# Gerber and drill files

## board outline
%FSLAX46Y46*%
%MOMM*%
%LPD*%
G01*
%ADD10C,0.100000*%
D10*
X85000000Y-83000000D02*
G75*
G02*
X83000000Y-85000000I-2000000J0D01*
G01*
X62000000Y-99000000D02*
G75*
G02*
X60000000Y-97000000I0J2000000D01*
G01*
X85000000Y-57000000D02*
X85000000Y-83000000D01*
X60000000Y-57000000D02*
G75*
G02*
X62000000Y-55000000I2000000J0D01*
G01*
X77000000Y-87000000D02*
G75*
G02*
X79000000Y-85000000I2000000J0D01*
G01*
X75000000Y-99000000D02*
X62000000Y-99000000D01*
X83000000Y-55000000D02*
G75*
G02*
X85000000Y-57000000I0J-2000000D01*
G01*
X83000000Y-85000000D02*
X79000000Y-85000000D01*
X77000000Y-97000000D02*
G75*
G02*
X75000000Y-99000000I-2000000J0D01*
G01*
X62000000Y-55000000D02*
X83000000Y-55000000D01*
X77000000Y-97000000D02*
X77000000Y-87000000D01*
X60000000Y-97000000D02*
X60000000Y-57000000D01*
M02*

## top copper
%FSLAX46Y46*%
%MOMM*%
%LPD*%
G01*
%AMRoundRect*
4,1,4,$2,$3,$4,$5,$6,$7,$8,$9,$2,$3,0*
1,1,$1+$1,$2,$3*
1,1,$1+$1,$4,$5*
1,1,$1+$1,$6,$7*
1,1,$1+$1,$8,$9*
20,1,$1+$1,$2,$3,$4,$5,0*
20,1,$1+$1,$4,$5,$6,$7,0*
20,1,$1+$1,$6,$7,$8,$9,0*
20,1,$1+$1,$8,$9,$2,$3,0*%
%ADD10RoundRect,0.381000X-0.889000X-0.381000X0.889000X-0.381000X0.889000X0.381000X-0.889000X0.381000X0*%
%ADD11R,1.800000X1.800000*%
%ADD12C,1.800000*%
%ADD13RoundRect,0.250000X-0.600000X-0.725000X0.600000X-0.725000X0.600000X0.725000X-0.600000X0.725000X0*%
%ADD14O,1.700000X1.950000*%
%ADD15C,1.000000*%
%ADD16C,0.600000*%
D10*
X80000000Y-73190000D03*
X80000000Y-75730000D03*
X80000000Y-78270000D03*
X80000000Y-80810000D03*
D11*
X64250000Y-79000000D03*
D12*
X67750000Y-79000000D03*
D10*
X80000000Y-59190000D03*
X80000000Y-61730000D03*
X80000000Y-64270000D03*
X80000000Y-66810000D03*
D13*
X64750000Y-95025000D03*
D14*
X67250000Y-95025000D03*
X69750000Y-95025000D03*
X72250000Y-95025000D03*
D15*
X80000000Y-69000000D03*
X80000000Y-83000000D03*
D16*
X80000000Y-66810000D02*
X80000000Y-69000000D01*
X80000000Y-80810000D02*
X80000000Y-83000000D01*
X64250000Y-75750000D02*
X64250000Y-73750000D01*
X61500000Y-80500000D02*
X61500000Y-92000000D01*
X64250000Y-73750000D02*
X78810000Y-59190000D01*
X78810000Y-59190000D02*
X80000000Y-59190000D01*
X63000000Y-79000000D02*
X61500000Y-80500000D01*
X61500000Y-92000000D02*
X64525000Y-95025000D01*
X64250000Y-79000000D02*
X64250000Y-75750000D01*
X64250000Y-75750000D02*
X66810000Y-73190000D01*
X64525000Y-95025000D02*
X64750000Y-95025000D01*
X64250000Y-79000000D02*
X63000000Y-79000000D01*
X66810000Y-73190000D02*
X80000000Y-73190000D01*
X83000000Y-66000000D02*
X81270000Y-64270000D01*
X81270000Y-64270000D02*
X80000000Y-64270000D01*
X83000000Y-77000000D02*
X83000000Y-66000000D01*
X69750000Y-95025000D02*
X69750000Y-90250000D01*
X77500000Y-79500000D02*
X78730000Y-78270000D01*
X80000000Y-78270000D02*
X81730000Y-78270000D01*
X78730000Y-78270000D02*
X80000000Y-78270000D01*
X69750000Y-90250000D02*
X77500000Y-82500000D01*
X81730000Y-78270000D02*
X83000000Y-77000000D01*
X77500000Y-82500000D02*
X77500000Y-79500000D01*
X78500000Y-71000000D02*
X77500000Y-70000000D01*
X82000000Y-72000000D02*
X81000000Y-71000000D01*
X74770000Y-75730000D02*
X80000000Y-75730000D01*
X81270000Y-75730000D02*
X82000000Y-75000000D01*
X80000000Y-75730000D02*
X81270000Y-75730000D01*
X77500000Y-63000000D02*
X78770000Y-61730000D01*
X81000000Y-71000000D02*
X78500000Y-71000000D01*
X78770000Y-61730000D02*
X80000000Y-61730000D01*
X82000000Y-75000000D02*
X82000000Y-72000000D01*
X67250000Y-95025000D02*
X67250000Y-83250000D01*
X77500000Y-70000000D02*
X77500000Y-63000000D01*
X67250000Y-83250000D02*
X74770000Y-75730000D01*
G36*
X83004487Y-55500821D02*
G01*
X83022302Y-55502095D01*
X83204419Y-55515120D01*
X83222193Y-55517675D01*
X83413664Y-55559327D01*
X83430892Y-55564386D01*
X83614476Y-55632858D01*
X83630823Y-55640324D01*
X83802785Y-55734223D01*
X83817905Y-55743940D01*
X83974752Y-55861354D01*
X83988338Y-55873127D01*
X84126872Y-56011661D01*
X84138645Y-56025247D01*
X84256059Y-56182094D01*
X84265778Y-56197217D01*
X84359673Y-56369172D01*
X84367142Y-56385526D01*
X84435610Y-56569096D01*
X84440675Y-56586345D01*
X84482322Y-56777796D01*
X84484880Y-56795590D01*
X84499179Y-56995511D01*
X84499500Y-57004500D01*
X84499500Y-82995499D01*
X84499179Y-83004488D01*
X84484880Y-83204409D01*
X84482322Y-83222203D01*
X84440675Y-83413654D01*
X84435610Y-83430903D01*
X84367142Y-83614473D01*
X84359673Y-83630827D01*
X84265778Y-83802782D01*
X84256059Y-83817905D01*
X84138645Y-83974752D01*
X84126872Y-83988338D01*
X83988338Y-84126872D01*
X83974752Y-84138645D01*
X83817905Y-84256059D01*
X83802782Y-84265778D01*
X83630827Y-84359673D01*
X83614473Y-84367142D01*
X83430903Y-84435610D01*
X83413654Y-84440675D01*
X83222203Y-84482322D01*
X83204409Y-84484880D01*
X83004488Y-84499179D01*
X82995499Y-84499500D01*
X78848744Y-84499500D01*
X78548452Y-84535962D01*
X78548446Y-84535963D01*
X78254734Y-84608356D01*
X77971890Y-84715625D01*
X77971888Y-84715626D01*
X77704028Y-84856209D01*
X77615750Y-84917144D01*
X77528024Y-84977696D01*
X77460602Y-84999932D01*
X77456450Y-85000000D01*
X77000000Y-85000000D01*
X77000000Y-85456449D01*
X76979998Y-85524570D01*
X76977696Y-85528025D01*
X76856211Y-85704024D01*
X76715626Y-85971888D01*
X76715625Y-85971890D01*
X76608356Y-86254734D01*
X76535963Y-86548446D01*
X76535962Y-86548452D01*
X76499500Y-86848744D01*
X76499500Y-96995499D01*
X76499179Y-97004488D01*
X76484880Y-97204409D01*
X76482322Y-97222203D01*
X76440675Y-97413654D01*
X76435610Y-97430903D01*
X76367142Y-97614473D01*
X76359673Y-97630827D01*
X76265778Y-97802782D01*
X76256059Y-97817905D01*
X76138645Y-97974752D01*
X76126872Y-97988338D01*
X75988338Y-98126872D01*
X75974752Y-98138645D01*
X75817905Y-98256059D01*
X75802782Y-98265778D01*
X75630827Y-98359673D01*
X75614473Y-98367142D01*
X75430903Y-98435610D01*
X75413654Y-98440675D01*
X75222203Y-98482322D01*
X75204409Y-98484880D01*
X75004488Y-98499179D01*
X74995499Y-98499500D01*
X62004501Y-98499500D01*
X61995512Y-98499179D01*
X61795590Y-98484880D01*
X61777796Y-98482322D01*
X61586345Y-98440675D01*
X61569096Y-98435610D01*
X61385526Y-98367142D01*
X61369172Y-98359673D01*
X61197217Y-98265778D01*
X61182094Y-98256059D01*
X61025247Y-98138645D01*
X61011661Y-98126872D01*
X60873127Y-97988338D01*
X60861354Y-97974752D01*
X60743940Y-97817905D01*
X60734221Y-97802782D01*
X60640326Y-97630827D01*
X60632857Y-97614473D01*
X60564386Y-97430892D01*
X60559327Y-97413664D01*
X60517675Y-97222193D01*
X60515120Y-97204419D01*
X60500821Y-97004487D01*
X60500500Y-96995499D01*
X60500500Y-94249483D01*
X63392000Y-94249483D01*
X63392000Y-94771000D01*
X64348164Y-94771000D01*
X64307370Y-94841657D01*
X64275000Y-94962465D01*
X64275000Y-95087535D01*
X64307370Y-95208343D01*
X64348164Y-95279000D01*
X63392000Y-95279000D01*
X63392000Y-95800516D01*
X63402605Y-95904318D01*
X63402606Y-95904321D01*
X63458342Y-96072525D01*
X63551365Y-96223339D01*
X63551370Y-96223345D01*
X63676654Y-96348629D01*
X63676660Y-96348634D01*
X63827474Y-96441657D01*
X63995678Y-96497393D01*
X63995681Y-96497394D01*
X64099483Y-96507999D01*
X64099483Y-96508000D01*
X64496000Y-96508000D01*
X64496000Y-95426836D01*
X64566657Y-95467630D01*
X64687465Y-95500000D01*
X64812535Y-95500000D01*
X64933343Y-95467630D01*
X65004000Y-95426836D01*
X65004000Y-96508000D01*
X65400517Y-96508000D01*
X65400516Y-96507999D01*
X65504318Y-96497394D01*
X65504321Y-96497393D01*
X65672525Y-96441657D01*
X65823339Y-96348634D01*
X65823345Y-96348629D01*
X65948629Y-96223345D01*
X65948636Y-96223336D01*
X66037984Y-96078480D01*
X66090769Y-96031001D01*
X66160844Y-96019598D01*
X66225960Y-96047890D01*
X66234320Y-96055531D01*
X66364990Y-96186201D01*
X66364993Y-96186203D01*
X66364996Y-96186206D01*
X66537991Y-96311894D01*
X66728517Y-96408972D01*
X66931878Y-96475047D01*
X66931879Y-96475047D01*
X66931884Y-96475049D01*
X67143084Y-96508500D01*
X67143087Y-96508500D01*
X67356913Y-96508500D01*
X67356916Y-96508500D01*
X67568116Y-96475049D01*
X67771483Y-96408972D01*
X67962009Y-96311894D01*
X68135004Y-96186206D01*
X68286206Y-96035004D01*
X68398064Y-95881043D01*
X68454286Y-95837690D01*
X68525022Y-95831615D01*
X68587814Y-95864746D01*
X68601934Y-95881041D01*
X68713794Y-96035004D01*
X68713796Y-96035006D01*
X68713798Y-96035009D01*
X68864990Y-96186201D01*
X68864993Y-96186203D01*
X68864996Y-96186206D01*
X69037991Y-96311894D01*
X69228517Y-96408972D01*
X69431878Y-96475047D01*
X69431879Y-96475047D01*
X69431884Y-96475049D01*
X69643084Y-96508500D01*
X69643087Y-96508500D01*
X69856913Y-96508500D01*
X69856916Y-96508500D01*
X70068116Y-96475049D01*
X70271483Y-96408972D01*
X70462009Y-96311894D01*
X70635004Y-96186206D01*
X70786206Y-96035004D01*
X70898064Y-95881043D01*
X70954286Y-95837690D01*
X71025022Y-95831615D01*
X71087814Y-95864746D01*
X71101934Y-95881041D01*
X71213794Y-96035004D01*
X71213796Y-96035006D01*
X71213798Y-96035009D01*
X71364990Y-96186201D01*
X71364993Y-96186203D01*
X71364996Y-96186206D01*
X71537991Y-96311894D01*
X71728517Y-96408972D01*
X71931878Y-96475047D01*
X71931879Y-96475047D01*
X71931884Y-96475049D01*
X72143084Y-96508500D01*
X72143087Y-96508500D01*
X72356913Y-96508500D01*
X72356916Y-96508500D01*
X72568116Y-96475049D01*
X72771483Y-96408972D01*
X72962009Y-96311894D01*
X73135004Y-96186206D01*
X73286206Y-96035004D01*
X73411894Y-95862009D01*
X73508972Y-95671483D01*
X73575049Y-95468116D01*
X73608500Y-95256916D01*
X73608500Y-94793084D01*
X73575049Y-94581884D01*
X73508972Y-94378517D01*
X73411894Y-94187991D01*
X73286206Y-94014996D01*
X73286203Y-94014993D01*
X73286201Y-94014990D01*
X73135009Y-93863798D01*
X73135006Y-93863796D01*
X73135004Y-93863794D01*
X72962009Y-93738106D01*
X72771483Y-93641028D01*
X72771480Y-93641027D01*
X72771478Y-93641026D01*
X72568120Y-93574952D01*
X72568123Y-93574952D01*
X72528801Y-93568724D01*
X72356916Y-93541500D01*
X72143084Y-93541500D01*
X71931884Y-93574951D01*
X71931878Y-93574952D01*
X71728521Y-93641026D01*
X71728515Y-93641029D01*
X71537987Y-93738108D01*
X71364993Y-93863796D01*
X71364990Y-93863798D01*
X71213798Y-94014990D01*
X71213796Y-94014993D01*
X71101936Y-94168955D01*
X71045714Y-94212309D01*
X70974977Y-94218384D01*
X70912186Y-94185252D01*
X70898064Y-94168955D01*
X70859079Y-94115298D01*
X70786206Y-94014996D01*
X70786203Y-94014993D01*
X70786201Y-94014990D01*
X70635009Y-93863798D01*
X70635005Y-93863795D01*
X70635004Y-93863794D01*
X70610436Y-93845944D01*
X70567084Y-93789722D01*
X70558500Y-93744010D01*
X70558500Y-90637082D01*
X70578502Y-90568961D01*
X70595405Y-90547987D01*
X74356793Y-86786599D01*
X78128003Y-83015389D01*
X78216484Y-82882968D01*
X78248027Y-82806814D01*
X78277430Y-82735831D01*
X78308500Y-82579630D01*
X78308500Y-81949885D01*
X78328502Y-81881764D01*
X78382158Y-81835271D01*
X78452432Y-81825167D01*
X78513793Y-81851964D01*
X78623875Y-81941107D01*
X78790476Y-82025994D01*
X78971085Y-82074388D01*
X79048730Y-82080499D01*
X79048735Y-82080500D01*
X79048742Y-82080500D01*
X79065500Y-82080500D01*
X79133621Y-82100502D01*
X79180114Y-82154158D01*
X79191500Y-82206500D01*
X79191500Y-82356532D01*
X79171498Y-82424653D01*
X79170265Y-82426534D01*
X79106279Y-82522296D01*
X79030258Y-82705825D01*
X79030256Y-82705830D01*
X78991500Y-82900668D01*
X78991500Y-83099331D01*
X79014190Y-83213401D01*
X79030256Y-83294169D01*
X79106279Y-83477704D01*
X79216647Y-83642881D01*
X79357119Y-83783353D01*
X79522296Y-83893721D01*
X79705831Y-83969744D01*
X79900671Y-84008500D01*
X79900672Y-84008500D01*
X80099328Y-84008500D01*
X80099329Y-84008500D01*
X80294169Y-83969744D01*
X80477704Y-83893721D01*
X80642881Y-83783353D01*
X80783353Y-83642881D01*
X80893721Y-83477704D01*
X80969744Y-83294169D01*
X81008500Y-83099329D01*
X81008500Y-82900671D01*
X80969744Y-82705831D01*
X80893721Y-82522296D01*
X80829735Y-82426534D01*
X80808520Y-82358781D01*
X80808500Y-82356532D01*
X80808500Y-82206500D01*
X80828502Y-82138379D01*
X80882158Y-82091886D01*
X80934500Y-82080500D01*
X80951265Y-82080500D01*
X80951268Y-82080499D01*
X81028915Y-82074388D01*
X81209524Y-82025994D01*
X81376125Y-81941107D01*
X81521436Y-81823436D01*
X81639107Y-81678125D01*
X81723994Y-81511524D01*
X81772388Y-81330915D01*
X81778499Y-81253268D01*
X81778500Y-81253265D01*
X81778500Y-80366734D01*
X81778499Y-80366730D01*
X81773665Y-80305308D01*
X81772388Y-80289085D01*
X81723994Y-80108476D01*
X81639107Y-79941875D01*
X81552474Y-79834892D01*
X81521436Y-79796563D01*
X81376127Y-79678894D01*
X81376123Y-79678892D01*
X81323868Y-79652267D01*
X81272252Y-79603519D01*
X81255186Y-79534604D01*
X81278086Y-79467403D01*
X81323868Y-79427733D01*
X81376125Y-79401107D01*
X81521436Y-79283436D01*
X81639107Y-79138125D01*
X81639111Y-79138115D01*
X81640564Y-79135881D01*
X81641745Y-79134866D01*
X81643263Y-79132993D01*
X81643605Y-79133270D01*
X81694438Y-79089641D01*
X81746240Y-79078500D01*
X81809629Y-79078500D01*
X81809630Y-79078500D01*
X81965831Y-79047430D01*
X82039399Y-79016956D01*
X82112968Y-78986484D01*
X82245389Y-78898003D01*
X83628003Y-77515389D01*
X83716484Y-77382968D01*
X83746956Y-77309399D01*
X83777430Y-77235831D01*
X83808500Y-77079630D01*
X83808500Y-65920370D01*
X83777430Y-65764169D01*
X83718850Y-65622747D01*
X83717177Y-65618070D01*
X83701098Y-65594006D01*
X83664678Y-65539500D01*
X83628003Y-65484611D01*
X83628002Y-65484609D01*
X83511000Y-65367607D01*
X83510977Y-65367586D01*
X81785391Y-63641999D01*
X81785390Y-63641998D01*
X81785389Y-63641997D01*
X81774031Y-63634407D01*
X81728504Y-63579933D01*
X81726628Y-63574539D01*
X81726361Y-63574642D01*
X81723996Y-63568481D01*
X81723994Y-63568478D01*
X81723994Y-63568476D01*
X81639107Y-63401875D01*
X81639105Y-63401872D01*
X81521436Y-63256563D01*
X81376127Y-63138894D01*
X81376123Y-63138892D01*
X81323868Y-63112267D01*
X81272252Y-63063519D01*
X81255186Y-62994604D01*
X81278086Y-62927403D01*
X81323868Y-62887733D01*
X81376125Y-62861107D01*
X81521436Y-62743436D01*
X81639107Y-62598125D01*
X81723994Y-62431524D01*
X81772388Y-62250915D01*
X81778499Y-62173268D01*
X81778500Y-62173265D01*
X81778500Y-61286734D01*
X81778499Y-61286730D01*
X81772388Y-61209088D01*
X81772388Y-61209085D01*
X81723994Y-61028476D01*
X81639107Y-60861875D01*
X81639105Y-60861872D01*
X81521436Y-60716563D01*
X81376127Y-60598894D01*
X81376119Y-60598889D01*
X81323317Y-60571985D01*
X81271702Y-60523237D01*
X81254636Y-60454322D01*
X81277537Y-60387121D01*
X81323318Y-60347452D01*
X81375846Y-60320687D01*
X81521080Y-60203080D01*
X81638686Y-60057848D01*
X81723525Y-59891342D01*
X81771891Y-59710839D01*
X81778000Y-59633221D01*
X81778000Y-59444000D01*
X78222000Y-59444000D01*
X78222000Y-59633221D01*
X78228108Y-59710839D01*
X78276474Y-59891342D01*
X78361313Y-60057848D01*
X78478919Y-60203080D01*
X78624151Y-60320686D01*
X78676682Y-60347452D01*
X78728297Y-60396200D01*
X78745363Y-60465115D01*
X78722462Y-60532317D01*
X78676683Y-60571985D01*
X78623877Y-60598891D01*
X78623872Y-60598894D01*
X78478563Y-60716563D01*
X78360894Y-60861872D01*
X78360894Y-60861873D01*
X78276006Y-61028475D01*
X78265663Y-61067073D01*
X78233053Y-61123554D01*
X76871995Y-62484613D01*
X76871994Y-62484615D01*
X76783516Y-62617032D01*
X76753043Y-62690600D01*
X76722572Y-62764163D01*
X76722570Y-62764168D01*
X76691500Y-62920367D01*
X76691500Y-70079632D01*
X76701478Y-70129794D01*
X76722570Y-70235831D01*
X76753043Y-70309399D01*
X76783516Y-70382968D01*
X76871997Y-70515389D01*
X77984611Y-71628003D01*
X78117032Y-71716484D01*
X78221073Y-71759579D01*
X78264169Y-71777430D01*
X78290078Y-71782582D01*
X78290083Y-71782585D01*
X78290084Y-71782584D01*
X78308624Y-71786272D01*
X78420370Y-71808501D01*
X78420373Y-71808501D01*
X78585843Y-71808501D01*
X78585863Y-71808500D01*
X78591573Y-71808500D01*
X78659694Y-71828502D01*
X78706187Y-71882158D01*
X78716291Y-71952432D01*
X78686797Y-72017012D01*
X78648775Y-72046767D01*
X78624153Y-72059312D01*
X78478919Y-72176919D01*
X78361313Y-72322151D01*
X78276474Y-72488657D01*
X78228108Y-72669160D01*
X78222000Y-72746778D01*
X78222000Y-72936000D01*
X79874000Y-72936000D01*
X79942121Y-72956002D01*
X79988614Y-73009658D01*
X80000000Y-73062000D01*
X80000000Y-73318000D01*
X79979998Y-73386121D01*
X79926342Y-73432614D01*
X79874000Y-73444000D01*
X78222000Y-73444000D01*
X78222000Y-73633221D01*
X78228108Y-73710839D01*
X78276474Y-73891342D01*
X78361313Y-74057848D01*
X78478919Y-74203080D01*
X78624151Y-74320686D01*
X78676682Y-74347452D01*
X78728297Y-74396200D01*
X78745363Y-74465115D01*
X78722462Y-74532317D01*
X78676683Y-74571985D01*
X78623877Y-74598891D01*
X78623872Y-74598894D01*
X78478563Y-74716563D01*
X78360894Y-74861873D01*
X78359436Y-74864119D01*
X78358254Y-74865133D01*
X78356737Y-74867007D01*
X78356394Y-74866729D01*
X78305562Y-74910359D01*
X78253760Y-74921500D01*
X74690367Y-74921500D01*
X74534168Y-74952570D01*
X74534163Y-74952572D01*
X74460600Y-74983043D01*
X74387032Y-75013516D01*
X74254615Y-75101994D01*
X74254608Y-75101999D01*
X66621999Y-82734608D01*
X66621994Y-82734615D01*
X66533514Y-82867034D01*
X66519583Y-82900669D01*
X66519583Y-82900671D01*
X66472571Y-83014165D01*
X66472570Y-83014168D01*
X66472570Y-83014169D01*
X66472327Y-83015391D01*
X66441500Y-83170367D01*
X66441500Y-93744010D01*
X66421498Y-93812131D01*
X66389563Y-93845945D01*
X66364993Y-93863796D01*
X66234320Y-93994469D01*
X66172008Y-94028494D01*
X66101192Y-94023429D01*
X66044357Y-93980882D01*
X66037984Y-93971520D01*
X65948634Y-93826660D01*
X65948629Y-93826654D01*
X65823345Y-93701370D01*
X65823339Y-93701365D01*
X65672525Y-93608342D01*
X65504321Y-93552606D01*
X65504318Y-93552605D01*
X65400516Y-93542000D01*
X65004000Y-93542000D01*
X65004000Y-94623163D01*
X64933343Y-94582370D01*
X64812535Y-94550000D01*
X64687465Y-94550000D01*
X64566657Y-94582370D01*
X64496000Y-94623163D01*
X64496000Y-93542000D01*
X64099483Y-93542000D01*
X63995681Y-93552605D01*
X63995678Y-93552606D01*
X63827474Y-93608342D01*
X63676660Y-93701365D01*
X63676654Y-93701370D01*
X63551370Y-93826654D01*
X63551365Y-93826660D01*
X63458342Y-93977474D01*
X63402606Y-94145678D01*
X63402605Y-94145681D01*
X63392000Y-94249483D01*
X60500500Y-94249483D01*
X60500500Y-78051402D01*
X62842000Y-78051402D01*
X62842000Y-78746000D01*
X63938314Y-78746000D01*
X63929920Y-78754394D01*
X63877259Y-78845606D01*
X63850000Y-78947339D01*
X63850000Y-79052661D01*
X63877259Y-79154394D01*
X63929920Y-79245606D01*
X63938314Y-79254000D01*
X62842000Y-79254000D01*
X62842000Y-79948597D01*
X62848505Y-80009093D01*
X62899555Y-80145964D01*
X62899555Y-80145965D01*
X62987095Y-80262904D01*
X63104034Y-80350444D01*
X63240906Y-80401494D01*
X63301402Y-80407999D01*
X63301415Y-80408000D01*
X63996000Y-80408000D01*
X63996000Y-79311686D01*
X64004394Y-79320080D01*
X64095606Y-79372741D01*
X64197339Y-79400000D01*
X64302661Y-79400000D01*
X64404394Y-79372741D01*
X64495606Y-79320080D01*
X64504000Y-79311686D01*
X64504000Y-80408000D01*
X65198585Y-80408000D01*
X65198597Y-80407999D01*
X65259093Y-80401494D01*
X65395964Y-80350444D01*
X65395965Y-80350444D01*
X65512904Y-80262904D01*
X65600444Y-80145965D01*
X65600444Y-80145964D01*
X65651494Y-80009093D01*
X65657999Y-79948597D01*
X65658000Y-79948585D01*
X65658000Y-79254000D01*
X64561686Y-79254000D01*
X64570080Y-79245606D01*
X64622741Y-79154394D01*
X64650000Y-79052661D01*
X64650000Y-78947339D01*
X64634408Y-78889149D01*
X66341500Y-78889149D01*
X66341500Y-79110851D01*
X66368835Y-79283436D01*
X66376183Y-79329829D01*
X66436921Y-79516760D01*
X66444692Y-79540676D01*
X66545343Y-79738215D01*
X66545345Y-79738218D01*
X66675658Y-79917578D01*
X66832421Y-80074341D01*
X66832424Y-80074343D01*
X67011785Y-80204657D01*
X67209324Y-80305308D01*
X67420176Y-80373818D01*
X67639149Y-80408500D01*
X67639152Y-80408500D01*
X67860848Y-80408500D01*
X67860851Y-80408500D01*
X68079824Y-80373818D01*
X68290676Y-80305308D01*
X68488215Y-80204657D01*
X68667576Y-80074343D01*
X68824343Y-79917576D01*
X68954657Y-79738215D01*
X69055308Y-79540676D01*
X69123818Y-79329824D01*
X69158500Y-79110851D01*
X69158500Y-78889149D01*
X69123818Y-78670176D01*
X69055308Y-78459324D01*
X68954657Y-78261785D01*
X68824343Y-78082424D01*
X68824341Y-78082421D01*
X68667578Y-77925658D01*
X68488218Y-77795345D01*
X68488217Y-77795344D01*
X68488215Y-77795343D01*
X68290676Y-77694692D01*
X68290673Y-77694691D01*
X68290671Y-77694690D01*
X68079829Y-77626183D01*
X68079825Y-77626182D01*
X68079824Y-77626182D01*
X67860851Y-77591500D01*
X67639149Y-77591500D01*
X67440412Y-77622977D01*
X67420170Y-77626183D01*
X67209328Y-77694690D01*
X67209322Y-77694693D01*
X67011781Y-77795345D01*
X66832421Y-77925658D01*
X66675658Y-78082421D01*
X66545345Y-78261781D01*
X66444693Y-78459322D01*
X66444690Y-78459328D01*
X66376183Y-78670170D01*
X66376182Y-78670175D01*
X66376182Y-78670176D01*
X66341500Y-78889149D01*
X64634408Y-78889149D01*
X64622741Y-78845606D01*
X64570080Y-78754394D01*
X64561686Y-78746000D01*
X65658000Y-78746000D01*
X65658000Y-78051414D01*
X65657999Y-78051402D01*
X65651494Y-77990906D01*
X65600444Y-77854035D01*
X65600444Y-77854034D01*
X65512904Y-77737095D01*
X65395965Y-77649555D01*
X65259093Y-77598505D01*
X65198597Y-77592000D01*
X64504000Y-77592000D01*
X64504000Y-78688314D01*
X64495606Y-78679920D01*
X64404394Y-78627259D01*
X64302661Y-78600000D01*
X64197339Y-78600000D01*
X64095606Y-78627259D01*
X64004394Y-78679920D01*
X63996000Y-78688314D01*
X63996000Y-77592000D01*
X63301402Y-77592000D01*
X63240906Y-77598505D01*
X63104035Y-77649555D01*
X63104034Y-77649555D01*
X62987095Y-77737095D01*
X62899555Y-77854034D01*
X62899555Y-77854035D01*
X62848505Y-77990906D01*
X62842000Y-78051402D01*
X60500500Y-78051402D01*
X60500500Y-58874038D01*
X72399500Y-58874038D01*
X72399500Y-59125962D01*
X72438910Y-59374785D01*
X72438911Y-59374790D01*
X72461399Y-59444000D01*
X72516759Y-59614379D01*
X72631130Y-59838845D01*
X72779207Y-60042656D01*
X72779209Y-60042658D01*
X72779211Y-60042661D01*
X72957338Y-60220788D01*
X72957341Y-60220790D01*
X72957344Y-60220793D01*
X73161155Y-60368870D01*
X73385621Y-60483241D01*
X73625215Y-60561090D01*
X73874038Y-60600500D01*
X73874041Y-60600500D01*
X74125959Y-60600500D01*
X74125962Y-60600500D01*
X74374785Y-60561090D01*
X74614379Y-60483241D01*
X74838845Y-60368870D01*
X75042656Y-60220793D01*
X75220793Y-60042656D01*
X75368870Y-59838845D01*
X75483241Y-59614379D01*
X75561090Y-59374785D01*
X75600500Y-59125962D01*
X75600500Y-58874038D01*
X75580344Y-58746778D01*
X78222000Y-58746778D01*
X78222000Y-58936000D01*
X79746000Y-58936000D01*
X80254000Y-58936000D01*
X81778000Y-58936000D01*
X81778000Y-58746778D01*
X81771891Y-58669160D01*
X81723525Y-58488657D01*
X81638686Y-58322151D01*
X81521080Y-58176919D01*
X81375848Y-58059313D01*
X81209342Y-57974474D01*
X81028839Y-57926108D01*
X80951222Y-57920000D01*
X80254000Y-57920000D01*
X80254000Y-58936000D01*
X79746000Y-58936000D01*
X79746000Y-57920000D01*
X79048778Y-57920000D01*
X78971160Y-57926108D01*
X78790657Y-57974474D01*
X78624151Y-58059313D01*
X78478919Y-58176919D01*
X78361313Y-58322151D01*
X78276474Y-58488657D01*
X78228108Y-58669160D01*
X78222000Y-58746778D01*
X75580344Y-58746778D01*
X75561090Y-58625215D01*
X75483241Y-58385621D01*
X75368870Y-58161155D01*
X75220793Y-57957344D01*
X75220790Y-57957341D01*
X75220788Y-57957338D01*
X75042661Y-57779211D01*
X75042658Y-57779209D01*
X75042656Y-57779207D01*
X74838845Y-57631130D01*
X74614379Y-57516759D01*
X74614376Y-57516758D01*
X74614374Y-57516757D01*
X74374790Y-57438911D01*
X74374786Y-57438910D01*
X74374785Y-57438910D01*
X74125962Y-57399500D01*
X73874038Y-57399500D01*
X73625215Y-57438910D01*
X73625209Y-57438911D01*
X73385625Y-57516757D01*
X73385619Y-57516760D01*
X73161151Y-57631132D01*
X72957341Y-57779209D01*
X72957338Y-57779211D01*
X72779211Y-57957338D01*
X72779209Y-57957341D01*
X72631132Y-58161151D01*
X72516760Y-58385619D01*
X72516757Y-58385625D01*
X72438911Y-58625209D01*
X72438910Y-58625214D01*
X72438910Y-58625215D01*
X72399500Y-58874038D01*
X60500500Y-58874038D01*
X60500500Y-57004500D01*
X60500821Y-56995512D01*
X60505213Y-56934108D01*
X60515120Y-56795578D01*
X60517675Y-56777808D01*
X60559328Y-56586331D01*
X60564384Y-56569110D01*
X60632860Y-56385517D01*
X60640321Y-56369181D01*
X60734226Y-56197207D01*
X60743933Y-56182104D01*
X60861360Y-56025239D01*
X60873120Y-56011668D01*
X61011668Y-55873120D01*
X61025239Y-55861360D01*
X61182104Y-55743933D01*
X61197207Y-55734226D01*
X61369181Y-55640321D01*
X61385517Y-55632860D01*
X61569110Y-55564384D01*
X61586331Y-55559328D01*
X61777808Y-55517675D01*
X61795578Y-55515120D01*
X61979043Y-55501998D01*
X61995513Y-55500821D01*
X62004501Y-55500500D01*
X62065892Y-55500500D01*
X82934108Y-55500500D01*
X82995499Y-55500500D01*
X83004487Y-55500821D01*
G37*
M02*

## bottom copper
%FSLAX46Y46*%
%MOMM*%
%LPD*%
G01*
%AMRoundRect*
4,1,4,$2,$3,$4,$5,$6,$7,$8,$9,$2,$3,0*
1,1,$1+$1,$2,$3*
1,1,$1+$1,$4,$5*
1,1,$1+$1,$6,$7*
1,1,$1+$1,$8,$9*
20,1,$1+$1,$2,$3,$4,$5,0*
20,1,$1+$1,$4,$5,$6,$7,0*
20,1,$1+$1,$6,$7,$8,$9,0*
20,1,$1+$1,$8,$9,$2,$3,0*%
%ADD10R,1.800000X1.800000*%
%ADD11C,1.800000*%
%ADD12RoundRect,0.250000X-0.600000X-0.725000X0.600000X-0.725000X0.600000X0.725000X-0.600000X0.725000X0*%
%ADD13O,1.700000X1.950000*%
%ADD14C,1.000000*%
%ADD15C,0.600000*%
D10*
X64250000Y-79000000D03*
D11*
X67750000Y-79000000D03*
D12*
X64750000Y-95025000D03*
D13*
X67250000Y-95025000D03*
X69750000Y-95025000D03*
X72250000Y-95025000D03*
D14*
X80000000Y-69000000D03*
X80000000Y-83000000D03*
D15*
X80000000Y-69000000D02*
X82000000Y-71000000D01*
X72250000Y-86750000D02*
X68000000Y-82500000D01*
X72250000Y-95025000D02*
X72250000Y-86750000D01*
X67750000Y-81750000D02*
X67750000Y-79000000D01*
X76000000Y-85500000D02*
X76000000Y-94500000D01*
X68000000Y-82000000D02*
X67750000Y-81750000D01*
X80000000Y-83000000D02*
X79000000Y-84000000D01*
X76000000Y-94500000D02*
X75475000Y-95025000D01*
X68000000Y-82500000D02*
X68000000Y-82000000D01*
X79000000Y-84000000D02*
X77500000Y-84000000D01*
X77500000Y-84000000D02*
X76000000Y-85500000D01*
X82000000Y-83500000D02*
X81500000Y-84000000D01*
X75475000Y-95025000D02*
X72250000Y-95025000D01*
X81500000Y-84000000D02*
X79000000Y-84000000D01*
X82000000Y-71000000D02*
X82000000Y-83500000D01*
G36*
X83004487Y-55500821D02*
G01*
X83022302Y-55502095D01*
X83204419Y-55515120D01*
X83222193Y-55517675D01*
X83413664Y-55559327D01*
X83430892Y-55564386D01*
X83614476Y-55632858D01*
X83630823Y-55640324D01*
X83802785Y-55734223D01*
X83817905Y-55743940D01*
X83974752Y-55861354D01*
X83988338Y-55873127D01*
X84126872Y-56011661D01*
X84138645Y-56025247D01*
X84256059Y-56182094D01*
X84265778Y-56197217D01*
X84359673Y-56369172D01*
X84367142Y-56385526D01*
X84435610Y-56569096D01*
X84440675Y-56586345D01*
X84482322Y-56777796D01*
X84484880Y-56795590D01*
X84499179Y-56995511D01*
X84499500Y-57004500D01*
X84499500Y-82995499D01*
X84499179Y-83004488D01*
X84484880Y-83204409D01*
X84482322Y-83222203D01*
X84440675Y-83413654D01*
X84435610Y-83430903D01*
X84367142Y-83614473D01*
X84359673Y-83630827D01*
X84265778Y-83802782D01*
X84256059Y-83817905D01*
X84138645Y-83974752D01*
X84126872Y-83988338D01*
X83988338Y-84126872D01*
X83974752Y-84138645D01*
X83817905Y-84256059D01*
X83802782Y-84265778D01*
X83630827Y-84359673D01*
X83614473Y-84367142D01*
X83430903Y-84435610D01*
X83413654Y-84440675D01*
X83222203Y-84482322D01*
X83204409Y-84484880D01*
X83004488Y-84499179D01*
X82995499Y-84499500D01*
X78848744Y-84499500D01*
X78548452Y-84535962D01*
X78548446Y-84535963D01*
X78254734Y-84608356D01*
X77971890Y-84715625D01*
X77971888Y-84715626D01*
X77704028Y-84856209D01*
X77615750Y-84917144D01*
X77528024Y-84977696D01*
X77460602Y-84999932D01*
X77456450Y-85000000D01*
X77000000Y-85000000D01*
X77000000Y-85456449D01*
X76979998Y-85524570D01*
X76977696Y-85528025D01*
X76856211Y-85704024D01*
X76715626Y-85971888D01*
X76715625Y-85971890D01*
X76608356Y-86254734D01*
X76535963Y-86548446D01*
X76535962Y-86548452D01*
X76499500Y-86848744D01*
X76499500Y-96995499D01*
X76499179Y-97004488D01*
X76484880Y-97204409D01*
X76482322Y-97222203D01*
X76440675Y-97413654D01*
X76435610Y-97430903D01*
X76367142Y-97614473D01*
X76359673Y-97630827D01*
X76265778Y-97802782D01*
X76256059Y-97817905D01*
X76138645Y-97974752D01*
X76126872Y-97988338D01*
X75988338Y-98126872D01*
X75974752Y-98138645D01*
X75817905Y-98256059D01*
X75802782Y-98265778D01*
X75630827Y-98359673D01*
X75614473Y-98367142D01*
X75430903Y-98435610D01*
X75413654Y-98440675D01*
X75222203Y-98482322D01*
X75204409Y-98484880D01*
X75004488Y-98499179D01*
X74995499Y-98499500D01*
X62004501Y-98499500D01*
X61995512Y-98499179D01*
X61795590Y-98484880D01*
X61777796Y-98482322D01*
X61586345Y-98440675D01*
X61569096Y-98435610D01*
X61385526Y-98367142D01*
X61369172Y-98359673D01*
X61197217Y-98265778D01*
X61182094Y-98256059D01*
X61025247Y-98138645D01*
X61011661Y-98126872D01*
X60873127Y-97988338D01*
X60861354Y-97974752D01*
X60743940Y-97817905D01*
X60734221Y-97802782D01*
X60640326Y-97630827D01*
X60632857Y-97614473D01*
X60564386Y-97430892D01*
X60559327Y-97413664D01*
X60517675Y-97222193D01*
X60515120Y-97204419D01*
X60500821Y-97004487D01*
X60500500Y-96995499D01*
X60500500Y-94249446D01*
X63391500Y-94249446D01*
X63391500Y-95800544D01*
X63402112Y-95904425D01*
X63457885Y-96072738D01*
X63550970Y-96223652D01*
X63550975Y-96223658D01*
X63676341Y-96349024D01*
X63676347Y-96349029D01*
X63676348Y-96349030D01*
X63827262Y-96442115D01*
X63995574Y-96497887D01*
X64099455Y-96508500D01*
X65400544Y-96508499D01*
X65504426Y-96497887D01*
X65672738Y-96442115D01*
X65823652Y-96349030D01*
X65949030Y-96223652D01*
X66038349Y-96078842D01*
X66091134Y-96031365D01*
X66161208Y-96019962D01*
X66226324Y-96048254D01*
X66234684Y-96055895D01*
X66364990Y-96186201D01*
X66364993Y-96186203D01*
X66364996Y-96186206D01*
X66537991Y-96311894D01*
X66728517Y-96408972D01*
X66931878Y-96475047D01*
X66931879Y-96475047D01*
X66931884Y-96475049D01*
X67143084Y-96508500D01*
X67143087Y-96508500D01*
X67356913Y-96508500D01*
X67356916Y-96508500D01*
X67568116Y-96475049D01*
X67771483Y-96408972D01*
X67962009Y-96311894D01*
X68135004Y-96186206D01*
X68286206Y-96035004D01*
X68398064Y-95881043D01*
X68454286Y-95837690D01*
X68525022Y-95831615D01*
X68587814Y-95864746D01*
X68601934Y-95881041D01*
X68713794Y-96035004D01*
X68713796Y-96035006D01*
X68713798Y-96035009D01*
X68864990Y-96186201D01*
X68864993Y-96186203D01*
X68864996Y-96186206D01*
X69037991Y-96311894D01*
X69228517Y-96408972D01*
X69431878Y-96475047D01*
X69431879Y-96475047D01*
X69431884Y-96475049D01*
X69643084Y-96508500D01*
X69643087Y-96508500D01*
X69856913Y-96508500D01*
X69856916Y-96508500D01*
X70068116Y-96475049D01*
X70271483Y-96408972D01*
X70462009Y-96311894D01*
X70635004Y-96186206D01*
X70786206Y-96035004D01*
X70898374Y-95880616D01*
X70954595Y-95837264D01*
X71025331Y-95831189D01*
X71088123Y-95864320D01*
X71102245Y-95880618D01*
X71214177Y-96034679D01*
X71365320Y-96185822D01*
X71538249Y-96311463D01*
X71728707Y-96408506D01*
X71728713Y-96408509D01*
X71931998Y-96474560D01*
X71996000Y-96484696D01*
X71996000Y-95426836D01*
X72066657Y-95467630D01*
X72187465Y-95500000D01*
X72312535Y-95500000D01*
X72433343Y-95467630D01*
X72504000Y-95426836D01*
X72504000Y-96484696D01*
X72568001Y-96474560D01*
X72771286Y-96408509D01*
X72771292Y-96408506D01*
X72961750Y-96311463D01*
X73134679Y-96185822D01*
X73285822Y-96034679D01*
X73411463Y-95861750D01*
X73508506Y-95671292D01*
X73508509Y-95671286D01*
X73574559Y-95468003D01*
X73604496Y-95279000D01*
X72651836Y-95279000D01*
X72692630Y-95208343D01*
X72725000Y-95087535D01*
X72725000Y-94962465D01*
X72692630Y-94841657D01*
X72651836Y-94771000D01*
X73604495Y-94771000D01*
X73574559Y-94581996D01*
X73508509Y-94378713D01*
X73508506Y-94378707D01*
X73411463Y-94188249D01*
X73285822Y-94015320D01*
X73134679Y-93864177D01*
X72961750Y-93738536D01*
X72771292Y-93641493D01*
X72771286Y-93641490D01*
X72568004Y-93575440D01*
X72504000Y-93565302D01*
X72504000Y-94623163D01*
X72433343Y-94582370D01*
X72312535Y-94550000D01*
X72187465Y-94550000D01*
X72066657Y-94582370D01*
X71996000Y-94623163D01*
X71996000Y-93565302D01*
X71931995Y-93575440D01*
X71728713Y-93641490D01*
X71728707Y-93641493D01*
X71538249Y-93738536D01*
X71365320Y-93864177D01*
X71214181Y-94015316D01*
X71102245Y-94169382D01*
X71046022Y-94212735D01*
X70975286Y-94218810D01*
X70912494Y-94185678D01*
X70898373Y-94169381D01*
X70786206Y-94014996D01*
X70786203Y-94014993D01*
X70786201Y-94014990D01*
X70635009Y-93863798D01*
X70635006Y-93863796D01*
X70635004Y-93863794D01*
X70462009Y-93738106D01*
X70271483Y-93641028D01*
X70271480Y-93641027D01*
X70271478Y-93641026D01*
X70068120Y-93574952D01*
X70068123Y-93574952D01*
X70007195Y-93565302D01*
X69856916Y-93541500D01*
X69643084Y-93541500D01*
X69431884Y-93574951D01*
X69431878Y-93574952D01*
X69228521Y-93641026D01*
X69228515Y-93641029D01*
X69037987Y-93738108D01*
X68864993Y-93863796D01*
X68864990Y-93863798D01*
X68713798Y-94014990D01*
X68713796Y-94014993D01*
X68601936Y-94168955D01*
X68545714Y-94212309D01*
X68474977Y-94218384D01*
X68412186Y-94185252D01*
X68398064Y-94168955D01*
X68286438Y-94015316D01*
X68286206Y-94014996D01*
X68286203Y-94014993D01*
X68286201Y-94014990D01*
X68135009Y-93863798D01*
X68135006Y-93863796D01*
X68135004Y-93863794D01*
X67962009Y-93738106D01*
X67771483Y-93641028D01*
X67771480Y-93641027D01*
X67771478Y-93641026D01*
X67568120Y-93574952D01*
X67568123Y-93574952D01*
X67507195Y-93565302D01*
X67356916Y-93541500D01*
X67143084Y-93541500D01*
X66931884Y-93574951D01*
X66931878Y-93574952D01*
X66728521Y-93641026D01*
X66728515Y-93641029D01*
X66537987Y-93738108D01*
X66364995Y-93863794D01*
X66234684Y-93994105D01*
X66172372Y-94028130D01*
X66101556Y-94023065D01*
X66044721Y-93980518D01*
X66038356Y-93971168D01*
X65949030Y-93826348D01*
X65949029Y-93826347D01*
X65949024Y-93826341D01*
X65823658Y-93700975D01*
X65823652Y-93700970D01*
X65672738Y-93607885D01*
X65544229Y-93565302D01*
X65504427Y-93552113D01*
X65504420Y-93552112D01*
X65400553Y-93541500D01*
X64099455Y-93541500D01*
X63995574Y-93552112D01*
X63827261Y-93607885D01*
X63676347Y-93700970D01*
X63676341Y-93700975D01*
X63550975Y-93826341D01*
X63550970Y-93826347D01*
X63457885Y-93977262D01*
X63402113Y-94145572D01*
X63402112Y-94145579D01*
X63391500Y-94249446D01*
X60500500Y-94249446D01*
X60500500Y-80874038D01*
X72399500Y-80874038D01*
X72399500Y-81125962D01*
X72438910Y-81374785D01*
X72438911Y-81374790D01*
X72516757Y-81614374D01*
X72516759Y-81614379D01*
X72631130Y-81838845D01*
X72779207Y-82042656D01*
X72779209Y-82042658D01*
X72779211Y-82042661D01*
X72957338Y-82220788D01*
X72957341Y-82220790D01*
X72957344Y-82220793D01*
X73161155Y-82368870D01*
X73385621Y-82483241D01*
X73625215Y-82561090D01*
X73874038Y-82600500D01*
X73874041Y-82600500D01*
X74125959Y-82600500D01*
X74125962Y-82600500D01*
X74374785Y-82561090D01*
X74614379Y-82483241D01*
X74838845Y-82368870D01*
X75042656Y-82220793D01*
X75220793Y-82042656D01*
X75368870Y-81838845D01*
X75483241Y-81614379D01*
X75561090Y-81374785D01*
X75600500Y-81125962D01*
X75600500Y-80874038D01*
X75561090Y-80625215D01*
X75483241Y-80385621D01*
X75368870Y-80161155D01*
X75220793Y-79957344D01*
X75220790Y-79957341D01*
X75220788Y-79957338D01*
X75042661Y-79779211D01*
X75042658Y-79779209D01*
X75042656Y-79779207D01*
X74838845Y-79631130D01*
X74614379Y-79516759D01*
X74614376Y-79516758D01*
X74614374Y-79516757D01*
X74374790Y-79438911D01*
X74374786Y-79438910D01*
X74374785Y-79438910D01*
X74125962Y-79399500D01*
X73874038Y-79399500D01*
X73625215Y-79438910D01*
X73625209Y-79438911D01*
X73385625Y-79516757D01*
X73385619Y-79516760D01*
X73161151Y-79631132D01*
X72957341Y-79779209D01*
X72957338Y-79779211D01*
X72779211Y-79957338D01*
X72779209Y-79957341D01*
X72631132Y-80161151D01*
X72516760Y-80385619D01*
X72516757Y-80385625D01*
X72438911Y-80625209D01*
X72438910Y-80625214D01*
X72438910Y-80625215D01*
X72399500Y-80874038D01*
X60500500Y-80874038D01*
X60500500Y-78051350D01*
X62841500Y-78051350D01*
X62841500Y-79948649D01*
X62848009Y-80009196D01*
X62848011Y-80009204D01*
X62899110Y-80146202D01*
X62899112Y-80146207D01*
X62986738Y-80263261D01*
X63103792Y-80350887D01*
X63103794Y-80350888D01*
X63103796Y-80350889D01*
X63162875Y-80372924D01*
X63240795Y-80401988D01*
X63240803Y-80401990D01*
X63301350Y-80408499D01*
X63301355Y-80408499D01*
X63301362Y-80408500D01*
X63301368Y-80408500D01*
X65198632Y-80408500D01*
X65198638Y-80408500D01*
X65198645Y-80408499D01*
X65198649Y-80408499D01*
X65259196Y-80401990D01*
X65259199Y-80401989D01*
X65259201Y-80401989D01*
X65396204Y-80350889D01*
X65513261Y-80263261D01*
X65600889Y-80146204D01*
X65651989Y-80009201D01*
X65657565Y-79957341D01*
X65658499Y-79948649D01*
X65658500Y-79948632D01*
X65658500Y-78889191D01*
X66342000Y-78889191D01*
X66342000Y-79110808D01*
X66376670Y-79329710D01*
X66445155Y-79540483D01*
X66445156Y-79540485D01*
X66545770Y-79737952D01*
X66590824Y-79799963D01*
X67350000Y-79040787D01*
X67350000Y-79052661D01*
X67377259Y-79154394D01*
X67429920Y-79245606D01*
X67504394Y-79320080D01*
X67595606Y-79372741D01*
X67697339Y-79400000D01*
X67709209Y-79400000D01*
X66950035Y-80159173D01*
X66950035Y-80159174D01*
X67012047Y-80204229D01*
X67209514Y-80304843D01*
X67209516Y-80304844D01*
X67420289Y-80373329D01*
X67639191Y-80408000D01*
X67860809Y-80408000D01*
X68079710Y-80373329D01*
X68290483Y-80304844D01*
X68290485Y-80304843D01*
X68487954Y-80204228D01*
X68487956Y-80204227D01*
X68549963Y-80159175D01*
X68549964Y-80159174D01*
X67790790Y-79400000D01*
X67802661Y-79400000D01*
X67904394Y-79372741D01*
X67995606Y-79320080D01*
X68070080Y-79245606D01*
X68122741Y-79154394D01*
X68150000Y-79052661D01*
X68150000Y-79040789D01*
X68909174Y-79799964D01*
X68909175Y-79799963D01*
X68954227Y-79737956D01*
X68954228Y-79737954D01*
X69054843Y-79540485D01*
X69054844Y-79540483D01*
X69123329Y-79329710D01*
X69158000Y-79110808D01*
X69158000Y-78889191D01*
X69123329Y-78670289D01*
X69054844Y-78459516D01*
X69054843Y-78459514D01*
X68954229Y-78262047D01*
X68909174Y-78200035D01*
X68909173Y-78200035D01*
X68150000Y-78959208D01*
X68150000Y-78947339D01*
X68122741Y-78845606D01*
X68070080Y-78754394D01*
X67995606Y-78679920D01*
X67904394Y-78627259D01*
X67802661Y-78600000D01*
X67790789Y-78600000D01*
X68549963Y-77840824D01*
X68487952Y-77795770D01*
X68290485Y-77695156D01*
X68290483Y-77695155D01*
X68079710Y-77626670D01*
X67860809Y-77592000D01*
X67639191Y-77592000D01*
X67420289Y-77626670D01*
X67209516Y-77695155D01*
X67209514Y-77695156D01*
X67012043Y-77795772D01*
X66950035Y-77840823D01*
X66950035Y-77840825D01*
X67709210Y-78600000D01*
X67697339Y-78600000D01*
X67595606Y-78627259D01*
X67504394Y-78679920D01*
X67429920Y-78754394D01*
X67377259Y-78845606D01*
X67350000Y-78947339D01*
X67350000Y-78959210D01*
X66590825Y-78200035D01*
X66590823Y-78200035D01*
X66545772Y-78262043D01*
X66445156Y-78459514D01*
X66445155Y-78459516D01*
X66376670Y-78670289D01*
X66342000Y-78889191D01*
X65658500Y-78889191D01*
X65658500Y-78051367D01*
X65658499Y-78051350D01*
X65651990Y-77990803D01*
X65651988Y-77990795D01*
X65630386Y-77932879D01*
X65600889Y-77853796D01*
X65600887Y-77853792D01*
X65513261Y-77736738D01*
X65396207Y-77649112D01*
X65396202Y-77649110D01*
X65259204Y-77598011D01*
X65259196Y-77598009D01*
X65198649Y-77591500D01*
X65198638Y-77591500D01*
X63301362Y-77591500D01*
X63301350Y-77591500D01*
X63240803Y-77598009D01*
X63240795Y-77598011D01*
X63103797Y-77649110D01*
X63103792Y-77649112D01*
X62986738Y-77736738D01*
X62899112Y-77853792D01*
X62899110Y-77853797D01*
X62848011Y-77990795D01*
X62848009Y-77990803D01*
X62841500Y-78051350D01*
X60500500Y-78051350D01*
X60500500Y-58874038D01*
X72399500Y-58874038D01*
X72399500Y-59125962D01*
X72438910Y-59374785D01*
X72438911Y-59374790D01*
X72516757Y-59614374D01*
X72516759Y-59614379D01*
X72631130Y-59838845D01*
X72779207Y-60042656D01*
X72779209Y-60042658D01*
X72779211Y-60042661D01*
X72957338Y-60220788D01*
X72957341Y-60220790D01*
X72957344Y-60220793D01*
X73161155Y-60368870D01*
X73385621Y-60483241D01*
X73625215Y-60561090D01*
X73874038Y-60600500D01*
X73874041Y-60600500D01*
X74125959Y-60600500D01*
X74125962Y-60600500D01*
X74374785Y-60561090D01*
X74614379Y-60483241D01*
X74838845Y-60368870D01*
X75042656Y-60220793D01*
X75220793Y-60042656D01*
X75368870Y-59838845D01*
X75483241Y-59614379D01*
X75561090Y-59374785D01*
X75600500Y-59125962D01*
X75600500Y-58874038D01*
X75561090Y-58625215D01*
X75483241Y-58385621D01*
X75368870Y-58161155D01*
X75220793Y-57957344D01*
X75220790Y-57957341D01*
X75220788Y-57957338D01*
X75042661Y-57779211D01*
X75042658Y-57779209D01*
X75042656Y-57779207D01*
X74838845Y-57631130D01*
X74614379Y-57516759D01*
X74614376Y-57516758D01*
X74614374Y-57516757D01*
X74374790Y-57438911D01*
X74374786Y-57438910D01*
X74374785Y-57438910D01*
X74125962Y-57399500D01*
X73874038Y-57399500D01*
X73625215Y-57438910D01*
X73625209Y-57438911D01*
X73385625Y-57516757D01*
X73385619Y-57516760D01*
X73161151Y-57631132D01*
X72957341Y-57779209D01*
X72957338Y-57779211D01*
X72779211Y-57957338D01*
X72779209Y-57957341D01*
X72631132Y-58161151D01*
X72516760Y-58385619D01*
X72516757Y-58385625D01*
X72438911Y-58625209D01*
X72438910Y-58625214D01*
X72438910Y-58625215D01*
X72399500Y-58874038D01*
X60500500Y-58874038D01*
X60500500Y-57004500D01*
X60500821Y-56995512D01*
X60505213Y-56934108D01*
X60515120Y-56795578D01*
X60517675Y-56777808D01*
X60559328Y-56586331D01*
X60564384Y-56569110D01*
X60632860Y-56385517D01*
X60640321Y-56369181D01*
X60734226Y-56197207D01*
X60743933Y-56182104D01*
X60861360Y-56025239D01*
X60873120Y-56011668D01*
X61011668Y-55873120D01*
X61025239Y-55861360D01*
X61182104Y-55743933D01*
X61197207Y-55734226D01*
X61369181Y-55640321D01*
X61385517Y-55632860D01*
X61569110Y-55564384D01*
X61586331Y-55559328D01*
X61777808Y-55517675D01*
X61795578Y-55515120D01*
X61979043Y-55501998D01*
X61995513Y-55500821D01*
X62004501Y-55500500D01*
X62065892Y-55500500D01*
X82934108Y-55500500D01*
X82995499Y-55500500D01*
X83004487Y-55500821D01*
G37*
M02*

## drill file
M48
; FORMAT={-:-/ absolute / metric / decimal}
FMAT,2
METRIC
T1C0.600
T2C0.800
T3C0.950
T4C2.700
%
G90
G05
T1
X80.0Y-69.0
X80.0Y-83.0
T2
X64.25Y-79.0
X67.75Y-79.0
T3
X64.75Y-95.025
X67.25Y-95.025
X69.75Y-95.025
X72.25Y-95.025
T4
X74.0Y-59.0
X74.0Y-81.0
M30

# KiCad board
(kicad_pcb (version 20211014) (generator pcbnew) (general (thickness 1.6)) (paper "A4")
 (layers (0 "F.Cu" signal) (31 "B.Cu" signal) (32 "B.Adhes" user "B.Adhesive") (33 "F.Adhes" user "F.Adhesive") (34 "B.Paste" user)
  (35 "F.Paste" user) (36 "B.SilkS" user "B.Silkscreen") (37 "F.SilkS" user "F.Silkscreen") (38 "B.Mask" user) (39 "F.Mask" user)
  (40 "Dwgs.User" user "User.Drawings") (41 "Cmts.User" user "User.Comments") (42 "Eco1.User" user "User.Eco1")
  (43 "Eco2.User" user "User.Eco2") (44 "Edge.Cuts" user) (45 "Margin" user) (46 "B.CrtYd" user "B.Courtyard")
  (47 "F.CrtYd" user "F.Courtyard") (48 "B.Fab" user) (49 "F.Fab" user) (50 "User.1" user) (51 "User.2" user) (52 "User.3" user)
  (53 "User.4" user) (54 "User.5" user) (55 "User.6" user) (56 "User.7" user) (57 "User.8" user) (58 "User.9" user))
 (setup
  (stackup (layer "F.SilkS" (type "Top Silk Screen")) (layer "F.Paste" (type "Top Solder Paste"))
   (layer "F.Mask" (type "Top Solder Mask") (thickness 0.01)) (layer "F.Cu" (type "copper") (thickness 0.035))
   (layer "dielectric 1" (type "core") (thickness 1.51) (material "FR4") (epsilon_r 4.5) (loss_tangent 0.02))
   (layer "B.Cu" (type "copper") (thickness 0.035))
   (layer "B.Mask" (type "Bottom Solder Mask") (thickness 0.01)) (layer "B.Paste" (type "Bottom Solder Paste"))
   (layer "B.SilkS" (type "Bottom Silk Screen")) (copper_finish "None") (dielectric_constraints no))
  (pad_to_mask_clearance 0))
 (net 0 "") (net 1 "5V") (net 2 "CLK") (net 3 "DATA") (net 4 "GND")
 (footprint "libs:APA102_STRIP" (layer "F.Cu") (at 80 77)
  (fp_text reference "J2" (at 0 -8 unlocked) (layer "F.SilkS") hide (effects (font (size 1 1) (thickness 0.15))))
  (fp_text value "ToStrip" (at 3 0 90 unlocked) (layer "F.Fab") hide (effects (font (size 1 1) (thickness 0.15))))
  (pad "1" connect roundrect (at 0 -3.81) (size 2.54 1.524) (layers "F.Cu" "F.Mask") (roundrect_rratio 0.25) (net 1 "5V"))
  (pad "2" connect roundrect (at 0 -1.27) (size 2.54 1.524) (layers "F.Cu" "F.Mask") (roundrect_rratio 0.25) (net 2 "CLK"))
  (pad "3" connect roundrect (at 0 1.27) (size 2.54 1.524) (layers "F.Cu" "F.Mask") (roundrect_rratio 0.25) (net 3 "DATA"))
  (pad "4" connect roundrect (at 0 3.81) (size 2.54 1.524) (layers "F.Cu" "F.Mask") (roundrect_rratio 0.25) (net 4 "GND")))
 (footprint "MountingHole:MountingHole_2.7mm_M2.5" (layer "F.Cu") (at 74 81)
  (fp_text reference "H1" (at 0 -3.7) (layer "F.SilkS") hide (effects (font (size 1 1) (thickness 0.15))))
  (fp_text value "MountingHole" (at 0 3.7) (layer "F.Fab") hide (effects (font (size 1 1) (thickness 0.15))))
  (pad "" np_thru_hole circle (at 0 0) (size 2.7 2.7) (drill 2.7) (layers *.Cu *.Mask)))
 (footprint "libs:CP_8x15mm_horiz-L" (layer "F.Cu") (at 66 79 -90)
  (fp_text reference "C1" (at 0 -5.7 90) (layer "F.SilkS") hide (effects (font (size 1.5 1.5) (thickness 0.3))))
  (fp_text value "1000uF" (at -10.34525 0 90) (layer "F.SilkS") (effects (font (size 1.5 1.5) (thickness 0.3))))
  (pad "1" thru_hole rect locked (at 0 1.75 270) (size 1.8 1.8) (drill 0.8) (layers *.Cu *.Mask "F.SilkS") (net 1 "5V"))
  (pad "2" thru_hole circle locked (at 0 -1.75 270) (size 1.8 1.8) (drill 0.8) (layers *.Cu *.Mask "F.SilkS") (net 4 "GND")))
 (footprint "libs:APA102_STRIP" (layer "F.Cu") (at 80 63)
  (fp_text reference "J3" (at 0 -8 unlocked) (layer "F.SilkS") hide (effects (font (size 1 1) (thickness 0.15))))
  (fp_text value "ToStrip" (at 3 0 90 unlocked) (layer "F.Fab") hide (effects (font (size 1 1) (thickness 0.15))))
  (pad "1" connect roundrect (at 0 -3.81) (size 2.54 1.524) (layers "F.Cu" "F.Mask") (roundrect_rratio 0.25) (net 1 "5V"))
  (pad "2" connect roundrect (at 0 -1.27) (size 2.54 1.524) (layers "F.Cu" "F.Mask") (roundrect_rratio 0.25) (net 2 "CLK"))
  (pad "3" connect roundrect (at 0 1.27) (size 2.54 1.524) (layers "F.Cu" "F.Mask") (roundrect_rratio 0.25) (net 3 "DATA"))
  (pad "4" connect roundrect (at 0 3.81) (size 2.54 1.524) (layers "F.Cu" "F.Mask") (roundrect_rratio 0.25) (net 4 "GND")))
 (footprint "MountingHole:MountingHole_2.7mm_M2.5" (layer "F.Cu") (at 74 59)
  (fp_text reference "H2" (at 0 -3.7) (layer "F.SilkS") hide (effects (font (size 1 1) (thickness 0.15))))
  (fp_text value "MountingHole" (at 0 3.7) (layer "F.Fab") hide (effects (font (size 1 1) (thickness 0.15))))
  (pad "" np_thru_hole circle (at 0 0) (size 2.7 2.7) (drill 2.7) (layers *.Cu *.Mask)))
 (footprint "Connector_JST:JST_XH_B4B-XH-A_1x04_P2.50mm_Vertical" (layer "B.Cu") (at 64.75 95.025)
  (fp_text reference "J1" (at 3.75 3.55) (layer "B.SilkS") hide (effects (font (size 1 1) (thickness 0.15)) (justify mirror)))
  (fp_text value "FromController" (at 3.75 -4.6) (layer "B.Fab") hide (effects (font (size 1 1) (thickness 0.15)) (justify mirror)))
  (pad "1" thru_hole roundrect (at 0 0) (size 1.7 1.95) (drill 0.95) (layers *.Cu *.Mask) (roundrect_rratio 0.1470588235) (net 1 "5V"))
  (pad "2" thru_hole oval (at 2.5 0) (size 1.7 1.95) (drill 0.95) (layers *.Cu *.Mask) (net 2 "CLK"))
  (pad "3" thru_hole oval (at 5 0) (size 1.7 1.95) (drill 0.95) (layers *.Cu *.Mask) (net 3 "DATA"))
  (pad "4" thru_hole oval (at 7.5 0) (size 1.7 1.95) (drill 0.95) (layers *.Cu *.Mask) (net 4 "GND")))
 (gr_arc (start 85 83) (mid 84.414214 84.414214) (end 83 85) (layer "Edge.Cuts") (width 0.1))
 (gr_arc (start 62 99) (mid 60.585786 98.414214) (end 60 97) (layer "Edge.Cuts") (width 0.1))
 (gr_line (start 85 57) (end 85 83) (layer "Edge.Cuts") (width 0.1))
 (gr_arc (start 60 57) (mid 60.585786 55.585786) (end 62 55) (layer "Edge.Cuts") (width 0.1))
 (gr_arc (start 77 87) (mid 77.585786 85.585786) (end 79 85) (layer "Edge.Cuts") (width 0.1))
 (gr_line (start 75 99) (end 62 99) (layer "Edge.Cuts") (width 0.1))
 (gr_arc (start 83 55) (mid 84.414214 55.585786) (end 85 57) (layer "Edge.Cuts") (width 0.1))
 (gr_line (start 83 85) (end 79 85) (layer "Edge.Cuts") (width 0.1))
 (gr_arc (start 77 97) (mid 76.414214 98.414214) (end 75 99) (layer "Edge.Cuts") (width 0.1))
 (gr_line (start 62 55) (end 83 55) (layer "Edge.Cuts") (width 0.1))
 (gr_line (start 77 97) (end 77 87) (layer "Edge.Cuts") (width 0.1))
 (gr_line (start 60 97) (end 60 57) (layer "Edge.Cuts") (width 0.1))
 (segment (start 80 66.81) (end 80 69) (width 0.6) (layer "F.Cu") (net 4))
 (segment (start 80 80.81) (end 80 83) (width 0.6) (layer "F.Cu") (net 4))
 (via (at 80 69) (size 1) (drill 0.6) (layers "F.Cu" "B.Cu") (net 4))
 (via (at 80 83) (size 1) (drill 0.6) (layers "F.Cu" "B.Cu") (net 4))
 (segment (start 80 69) (end 82 71) (width 0.6) (layer "B.Cu") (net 4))
 (segment (start 72.25 86.75) (end 68 82.5) (width 0.6) (layer "B.Cu") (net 4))
 (segment (start 72.25 95.025) (end 72.25 86.75) (width 0.6) (layer "B.Cu") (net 4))
 (segment (start 67.75 81.75) (end 67.75 79) (width 0.6) (layer "B.Cu") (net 4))
 (segment (start 76 85.5) (end 76 94.5) (width 0.6) (layer "B.Cu") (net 4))
 (segment (start 68 82) (end 67.75 81.75) (width 0.6) (layer "B.Cu") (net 4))
 (segment (start 80 83) (end 79 84) (width 0.6) (layer "B.Cu") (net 4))
 (segment (start 76 94.5) (end 75.475 95.025) (width 0.6) (layer "B.Cu") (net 4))
 (segment (start 68 82.5) (end 68 82) (width 0.6) (layer "B.Cu") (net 4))
 (segment (start 79 84) (end 77.5 84) (width 0.6) (layer "B.Cu") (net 4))
 (segment (start 77.5 84) (end 76 85.5) (width 0.6) (layer "B.Cu") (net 4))
 (segment (start 82 83.5) (end 81.5 84) (width 0.6) (layer "B.Cu") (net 4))
 (segment (start 75.475 95.025) (end 72.25 95.025) (width 0.6) (layer "B.Cu") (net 4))
 (segment (start 81.5 84) (end 79 84) (width 0.6) (layer "B.Cu") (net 4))
 (segment (start 82 71) (end 82 83.5) (width 0.6) (layer "B.Cu") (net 4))
 (segment (start 64.25 75.75) (end 64.25 73.75) (width 0.6) (layer "F.Cu") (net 1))
 (segment (start 61.5 80.5) (end 61.5 92) (width 0.6) (layer "F.Cu") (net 1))
 (segment (start 64.25 73.75) (end 78.81 59.19) (width 0.6) (layer "F.Cu") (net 1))
 (segment (start 78.81 59.19) (end 80 59.19) (width 0.6) (layer "F.Cu") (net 1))
 (segment (start 63 79) (end 61.5 80.5) (width 0.6) (layer "F.Cu") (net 1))
 (segment (start 61.5 92) (end 64.525 95.025) (width 0.6) (layer "F.Cu") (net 1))
 (segment (start 64.25 79) (end 64.25 75.75) (width 0.6) (layer "F.Cu") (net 1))
 (segment (start 64.25 75.75) (end 66.81 73.19) (width 0.6) (layer "F.Cu") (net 1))
 (segment (start 64.525 95.025) (end 64.75 95.025) (width 0.6) (layer "F.Cu") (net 1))
 (segment (start 64.25 79) (end 63 79) (width 0.6) (layer "F.Cu") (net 1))
 (segment (start 66.81 73.19) (end 80 73.19) (width 0.6) (layer "F.Cu") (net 1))
 (segment (start 83 66) (end 81.27 64.27) (width 0.6) (layer "F.Cu") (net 3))
 (segment (start 81.27 64.27) (end 80 64.27) (width 0.6) (layer "F.Cu") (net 3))
 (segment (start 83 77) (end 83 66) (width 0.6) (layer "F.Cu") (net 3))
 (segment (start 69.75 95.025) (end 69.75 90.25) (width 0.6) (layer "F.Cu") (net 3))
 (segment (start 77.5 79.5) (end 78.73 78.27) (width 0.6) (layer "F.Cu") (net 3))
 (segment (start 80 78.27) (end 81.73 78.27) (width 0.6) (layer "F.Cu") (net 3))
 (segment (start 78.73 78.27) (end 80 78.27) (width 0.6) (layer "F.Cu") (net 3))
 (segment (start 69.75 90.25) (end 77.5 82.5) (width 0.6) (layer "F.Cu") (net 3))
 (segment (start 81.73 78.27) (end 83 77) (width 0.6) (layer "F.Cu") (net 3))
 (segment (start 77.5 82.5) (end 77.5 79.5) (width 0.6) (layer "F.Cu") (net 3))
 (segment (start 78.5 71) (end 77.5 70) (width 0.6) (layer "F.Cu") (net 2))
 (segment (start 82 72) (end 81 71) (width 0.6) (layer "F.Cu") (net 2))
 (segment (start 74.77 75.73) (end 80 75.73) (width 0.6) (layer "F.Cu") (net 2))
 (segment (start 81.27 75.73) (end 82 75) (width 0.6) (layer "F.Cu") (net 2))
 (segment (start 80 75.73) (end 81.27 75.73) (width 0.6) (layer "F.Cu") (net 2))
 (segment (start 77.5 63) (end 78.77 61.73) (width 0.6) (layer "F.Cu") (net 2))
 (segment (start 81 71) (end 78.5 71) (width 0.6) (layer "F.Cu") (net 2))
 (segment (start 78.77 61.73) (end 80 61.73) (width 0.6) (layer "F.Cu") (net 2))
 (segment (start 82 75) (end 82 72) (width 0.6) (layer "F.Cu") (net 2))
 (segment (start 67.25 95.025) (end 67.25 83.25) (width 0.6) (layer "F.Cu") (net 2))
 (segment (start 77.5 70) (end 77.5 63) (width 0.6) (layer "F.Cu") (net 2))
 (segment (start 67.25 83.25) (end 74.77 75.73) (width 0.6) (layer "F.Cu") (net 2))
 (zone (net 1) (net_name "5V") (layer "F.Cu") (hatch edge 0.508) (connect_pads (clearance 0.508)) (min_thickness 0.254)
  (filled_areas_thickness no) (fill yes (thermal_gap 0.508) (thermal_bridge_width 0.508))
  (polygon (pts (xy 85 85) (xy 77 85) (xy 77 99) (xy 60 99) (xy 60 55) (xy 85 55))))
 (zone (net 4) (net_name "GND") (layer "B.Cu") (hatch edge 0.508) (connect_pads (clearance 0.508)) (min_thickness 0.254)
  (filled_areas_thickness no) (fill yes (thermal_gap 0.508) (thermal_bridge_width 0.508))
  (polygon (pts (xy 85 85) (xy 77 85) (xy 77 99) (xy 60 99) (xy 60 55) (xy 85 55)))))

